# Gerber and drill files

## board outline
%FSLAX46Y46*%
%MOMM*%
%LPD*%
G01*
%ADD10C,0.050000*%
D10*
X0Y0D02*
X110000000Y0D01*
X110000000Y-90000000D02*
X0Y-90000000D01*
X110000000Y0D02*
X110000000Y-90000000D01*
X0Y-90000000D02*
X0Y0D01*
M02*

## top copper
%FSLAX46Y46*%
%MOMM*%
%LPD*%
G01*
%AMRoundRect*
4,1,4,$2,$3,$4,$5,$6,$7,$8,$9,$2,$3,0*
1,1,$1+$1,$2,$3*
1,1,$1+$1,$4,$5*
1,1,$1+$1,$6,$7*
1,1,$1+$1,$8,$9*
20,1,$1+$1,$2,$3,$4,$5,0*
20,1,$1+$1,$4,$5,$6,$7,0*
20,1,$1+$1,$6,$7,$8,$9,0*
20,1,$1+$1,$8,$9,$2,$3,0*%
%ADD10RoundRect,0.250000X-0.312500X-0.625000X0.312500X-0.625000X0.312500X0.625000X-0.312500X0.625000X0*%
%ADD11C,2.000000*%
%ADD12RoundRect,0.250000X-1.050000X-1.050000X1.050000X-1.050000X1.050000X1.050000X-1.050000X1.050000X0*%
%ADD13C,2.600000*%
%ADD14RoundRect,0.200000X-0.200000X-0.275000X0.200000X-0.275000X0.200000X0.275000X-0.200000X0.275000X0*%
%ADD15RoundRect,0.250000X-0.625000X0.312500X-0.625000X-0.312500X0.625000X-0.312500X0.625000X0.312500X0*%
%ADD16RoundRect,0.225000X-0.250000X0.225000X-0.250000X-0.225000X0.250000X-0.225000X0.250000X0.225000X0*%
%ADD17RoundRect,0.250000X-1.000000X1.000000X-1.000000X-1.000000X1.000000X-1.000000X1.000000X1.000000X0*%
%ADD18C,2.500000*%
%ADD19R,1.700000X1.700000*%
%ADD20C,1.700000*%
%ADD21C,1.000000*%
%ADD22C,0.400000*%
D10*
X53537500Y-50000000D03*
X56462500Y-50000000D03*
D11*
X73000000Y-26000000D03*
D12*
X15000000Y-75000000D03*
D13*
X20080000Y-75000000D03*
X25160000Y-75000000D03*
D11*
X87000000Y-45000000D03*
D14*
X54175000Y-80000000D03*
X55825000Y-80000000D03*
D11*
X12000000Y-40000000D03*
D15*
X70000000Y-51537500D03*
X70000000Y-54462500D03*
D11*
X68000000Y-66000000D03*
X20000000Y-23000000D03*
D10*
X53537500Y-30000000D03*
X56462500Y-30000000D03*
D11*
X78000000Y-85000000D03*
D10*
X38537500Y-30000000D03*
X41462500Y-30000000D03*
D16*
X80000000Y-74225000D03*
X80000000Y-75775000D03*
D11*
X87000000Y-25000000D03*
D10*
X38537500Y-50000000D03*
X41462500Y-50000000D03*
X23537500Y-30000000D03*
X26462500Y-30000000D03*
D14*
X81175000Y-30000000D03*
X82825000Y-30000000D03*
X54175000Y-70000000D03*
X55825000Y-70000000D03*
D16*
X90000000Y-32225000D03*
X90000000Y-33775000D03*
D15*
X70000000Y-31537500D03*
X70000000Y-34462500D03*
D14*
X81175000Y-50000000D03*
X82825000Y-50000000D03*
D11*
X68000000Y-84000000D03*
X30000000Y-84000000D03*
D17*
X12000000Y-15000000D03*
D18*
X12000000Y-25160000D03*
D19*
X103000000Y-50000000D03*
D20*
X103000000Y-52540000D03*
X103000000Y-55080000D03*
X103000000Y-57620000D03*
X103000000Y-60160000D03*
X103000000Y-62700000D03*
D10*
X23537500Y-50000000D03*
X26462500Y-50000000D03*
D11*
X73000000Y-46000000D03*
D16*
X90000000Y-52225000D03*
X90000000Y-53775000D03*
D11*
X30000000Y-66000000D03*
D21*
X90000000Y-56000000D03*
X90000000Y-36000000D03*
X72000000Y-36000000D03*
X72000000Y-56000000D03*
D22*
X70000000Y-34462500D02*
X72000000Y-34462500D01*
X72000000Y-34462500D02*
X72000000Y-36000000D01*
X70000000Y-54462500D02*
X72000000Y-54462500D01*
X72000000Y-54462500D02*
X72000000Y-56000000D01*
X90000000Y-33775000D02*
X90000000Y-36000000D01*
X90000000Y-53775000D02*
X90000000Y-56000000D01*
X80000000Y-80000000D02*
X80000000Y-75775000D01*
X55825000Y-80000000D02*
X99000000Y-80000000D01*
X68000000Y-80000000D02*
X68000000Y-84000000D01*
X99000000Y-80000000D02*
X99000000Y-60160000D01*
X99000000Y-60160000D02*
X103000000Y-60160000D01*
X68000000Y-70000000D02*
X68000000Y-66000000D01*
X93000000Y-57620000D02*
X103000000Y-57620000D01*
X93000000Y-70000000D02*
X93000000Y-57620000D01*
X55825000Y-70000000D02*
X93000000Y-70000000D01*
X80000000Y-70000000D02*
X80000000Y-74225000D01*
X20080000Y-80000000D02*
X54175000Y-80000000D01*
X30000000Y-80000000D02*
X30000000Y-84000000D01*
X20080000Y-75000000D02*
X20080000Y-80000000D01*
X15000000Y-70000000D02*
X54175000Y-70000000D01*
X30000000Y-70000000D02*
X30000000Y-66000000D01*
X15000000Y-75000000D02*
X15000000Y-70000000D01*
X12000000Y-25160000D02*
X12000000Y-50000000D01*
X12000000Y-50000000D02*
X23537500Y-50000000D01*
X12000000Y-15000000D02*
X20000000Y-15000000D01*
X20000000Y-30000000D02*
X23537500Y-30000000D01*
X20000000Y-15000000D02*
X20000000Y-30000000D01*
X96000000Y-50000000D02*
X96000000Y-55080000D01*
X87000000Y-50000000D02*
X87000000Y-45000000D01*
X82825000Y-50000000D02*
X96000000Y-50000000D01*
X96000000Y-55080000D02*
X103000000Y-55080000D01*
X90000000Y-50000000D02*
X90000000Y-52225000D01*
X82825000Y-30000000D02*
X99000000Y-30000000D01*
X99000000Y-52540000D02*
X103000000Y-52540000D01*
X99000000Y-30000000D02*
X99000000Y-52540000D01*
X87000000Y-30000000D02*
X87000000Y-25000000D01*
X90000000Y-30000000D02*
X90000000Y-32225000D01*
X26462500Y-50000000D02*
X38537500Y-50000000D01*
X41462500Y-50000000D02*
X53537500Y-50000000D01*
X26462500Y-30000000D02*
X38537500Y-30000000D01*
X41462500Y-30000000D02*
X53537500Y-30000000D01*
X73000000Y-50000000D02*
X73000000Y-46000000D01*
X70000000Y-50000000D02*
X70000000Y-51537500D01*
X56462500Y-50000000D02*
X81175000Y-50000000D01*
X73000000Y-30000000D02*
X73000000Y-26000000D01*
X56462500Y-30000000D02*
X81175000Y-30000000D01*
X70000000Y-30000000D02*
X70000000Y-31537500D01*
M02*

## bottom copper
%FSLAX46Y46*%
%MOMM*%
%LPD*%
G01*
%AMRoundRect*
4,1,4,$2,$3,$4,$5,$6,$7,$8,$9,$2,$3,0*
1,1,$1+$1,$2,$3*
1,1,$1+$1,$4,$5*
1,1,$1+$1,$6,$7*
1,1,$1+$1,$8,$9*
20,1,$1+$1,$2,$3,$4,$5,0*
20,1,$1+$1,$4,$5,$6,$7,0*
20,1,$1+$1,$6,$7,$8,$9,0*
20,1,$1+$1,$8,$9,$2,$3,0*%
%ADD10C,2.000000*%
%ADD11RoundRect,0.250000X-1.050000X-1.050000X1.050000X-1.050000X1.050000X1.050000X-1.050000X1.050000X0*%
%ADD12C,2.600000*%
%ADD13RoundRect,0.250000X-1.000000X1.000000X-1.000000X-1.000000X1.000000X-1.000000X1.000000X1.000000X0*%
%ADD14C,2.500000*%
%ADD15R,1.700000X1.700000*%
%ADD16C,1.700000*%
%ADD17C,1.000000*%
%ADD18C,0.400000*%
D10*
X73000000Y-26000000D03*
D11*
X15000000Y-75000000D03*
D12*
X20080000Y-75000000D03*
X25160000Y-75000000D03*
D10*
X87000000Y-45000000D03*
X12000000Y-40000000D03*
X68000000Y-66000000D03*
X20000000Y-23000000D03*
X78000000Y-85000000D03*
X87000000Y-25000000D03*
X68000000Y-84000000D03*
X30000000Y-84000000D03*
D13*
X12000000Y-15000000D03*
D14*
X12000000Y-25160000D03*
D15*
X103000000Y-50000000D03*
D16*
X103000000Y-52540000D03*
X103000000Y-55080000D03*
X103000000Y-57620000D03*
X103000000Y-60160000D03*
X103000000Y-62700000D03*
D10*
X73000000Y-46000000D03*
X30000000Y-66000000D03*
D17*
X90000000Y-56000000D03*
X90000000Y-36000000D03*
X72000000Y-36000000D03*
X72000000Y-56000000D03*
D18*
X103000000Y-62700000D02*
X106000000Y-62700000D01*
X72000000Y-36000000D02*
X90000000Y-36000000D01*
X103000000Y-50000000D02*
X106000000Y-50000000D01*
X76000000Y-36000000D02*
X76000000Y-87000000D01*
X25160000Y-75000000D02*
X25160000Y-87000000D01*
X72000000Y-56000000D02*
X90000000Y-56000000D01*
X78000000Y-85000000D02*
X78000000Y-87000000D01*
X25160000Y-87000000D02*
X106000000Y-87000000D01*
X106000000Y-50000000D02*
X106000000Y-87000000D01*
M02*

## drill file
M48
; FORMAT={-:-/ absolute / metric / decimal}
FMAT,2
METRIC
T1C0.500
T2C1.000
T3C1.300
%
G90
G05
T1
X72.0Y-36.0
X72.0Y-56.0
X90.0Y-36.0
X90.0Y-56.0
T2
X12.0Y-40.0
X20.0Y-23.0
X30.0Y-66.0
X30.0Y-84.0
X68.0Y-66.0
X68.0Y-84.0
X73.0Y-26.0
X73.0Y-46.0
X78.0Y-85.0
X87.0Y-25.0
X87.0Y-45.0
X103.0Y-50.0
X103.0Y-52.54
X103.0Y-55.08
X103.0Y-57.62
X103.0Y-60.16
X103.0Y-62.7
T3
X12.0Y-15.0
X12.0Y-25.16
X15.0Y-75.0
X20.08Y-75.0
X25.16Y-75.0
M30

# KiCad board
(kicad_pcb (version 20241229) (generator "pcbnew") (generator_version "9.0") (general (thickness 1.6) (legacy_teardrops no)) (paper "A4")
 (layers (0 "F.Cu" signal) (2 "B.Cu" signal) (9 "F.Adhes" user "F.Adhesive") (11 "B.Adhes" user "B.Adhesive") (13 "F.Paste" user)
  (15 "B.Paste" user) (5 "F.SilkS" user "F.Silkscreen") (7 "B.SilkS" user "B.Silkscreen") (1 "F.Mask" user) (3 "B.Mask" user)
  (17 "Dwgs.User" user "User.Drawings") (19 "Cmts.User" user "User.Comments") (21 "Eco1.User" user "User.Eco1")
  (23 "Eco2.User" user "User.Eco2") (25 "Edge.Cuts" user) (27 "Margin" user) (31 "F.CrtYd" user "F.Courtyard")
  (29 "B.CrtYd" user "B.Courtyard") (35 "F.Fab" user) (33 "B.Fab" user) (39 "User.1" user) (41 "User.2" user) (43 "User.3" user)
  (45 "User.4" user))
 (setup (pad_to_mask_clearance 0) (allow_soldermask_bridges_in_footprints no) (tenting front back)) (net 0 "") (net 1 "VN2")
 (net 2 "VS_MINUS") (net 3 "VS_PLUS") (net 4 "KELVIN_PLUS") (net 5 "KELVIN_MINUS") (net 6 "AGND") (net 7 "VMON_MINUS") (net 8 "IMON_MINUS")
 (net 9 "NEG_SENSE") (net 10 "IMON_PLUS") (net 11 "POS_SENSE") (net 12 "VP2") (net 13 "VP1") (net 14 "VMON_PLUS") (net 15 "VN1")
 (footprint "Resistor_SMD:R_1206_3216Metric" (layer "F.Cu") (at 55 50)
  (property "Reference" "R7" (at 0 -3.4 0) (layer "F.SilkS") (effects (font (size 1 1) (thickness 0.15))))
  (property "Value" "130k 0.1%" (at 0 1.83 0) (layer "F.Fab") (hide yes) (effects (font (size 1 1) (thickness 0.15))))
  (pad "1" smd roundrect (at -1.4625 0) (size 1.125 1.75) (layers "F.Cu" "F.Mask" "F.Paste") (roundrect_rratio 0.222222) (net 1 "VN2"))
  (pad "2" smd roundrect (at 1.4625 0) (size 1.125 1.75) (layers "F.Cu" "F.Mask" "F.Paste") (roundrect_rratio 0.222222) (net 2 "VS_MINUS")))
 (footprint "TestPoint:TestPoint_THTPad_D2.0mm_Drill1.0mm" (layer "F.Cu") (at 73 26)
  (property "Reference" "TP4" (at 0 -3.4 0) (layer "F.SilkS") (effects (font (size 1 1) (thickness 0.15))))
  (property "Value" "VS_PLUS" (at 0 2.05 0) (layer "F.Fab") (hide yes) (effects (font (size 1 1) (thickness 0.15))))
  (pad "1" thru_hole circle (at 0 0) (size 2 2) (drill 1) (layers "*.Cu" "*.Mask") (remove_unused_layers no) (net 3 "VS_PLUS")))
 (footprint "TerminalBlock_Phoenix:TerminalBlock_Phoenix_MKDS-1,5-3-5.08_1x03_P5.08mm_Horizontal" (layer "F.Cu") (at 15 75)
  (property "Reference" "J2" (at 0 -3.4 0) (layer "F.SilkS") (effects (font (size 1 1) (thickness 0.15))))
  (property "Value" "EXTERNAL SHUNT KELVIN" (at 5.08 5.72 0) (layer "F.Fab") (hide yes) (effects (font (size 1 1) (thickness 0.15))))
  (pad "1" thru_hole roundrect (at 0 0) (size 2.6 2.6) (drill 1.3) (layers "*.Cu" "*.Mask") (remove_unused_layers no)
   (roundrect_rratio 0.096154) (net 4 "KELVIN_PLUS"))
  (pad "2" thru_hole circle (at 5.08 0) (size 2.6 2.6) (drill 1.3) (layers "*.Cu" "*.Mask") (remove_unused_layers no) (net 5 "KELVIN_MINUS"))
  (pad "3" thru_hole circle (at 10.16 0) (size 2.6 2.6) (drill 1.3) (layers "*.Cu" "*.Mask") (remove_unused_layers no) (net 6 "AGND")))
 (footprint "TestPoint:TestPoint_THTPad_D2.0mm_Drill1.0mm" (layer "F.Cu") (at 87 45)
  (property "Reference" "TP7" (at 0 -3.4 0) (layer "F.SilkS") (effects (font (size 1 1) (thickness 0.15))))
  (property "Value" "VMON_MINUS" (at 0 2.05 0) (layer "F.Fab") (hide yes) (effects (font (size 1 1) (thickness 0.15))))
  (pad "1" thru_hole circle (at 0 0) (size 2 2) (drill 1) (layers "*.Cu" "*.Mask") (remove_unused_layers no) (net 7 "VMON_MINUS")))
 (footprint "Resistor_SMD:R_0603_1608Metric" (layer "F.Cu") (at 55 80)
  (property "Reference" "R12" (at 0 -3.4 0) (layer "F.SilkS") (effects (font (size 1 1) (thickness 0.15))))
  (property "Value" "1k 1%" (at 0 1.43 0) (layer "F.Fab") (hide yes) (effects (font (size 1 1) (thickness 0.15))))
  (pad "1" smd roundrect (at -0.825 0) (size 0.8 0.95) (layers "F.Cu" "F.Mask" "F.Paste") (roundrect_rratio 0.25) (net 5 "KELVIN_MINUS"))
  (pad "2" smd roundrect (at 0.825 0) (size 0.8 0.95) (layers "F.Cu" "F.Mask" "F.Paste") (roundrect_rratio 0.25) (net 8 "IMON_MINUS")))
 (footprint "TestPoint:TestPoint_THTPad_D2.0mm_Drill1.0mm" (layer "F.Cu") (at 12 40)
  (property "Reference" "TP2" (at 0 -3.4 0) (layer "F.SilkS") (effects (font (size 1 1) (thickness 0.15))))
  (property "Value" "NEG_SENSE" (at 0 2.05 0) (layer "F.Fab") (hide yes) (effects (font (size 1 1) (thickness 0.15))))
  (pad "1" thru_hole circle (at 0 0) (size 2 2) (drill 1) (layers "*.Cu" "*.Mask") (remove_unused_layers no) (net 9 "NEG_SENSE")))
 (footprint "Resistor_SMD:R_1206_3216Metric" (layer "F.Cu") (at 70 53 -90)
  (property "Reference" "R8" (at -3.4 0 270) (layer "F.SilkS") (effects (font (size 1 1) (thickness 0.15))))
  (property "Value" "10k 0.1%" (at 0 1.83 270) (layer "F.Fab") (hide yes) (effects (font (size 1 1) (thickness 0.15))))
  (pad "1" smd roundrect (at -1.4625 0 270) (size 1.125 1.75) (layers "F.Cu" "F.Mask" "F.Paste") (roundrect_rratio 0.222222)
   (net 2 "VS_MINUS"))
  (pad "2" smd roundrect (at 1.4625 0 270) (size 1.125 1.75) (layers "F.Cu" "F.Mask" "F.Paste") (roundrect_rratio 0.222222) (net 6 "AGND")))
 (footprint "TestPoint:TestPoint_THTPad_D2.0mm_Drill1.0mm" (layer "F.Cu") (at 68 66)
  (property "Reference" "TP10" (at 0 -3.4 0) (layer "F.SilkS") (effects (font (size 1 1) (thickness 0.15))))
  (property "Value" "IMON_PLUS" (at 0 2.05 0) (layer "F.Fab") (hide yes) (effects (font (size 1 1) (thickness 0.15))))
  (pad "1" thru_hole circle (at 0 0) (size 2 2) (drill 1) (layers "*.Cu" "*.Mask") (remove_unused_layers no) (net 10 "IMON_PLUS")))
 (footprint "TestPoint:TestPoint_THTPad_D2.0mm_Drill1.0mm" (layer "F.Cu") (at 20 23)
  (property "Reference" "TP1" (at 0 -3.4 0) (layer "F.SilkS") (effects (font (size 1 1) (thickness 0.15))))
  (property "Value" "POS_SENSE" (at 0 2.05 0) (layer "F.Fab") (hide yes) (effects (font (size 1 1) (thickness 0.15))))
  (pad "1" thru_hole circle (at 0 0) (size 2 2) (drill 1) (layers "*.Cu" "*.Mask") (remove_unused_layers no) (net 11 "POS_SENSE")))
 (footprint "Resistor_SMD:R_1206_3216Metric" (layer "F.Cu") (at 55 30)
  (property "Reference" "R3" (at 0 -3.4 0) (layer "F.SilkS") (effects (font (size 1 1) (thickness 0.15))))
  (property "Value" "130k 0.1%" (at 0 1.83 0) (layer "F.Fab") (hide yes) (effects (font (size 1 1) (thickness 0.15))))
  (pad "1" smd roundrect (at -1.4625 0) (size 1.125 1.75) (layers "F.Cu" "F.Mask" "F.Paste") (roundrect_rratio 0.222222) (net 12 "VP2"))
  (pad "2" smd roundrect (at 1.4625 0) (size 1.125 1.75) (layers "F.Cu" "F.Mask" "F.Paste") (roundrect_rratio 0.222222) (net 3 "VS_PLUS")))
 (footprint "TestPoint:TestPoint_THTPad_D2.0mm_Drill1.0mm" (layer "F.Cu") (at 78 85)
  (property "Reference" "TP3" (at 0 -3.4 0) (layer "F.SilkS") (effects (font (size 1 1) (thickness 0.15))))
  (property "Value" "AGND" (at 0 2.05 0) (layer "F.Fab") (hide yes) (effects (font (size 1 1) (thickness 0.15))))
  (pad "1" thru_hole circle (at 0 0) (size 2 2) (drill 1) (layers "*.Cu" "*.Mask") (remove_unused_layers no) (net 6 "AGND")))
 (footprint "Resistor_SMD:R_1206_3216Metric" (layer "F.Cu") (at 40 30)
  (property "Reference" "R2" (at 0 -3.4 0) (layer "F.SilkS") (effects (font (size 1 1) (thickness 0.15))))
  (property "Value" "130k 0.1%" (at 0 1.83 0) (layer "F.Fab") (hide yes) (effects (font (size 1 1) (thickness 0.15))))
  (pad "1" smd roundrect (at -1.4625 0) (size 1.125 1.75) (layers "F.Cu" "F.Mask" "F.Paste") (roundrect_rratio 0.222222) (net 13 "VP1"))
  (pad "2" smd roundrect (at 1.4625 0) (size 1.125 1.75) (layers "F.Cu" "F.Mask" "F.Paste") (roundrect_rratio 0.222222) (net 12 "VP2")))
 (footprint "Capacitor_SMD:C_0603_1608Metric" (layer "F.Cu") (at 80 75 -90)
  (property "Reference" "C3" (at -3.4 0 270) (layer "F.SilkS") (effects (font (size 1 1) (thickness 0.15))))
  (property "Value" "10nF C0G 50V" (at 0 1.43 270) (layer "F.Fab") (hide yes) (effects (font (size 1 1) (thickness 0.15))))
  (pad "1" smd roundrect (at -0.775 0 270) (size 0.9 0.95) (layers "F.Cu" "F.Mask" "F.Paste") (roundrect_rratio 0.25) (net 10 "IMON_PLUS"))
  (pad "2" smd roundrect (at 0.775 0 270) (size 0.9 0.95) (layers "F.Cu" "F.Mask" "F.Paste") (roundrect_rratio 0.25) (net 8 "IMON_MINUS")))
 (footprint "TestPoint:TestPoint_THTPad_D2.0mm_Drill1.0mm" (layer "F.Cu") (at 87 25)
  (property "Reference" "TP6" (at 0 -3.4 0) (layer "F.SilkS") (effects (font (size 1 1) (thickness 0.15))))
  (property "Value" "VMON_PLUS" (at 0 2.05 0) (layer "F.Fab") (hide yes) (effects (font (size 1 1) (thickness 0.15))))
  (pad "1" thru_hole circle (at 0 0) (size 2 2) (drill 1) (layers "*.Cu" "*.Mask") (remove_unused_layers no) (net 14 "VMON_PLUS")))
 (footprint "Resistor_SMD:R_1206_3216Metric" (layer "F.Cu") (at 40 50)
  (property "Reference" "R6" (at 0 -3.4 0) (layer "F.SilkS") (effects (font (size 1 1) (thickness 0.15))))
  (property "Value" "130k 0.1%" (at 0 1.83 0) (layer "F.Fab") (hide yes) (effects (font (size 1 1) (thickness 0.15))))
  (pad "1" smd roundrect (at -1.4625 0) (size 1.125 1.75) (layers "F.Cu" "F.Mask" "F.Paste") (roundrect_rratio 0.222222) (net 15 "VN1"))
  (pad "2" smd roundrect (at 1.4625 0) (size 1.125 1.75) (layers "F.Cu" "F.Mask" "F.Paste") (roundrect_rratio 0.222222) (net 1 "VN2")))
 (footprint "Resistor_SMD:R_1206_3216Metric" (layer "F.Cu") (at 25 30)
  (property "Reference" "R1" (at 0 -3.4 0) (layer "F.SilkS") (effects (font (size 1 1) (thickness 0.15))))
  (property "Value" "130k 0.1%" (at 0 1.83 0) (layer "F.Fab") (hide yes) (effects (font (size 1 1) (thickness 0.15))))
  (pad "1" smd roundrect (at -1.4625 0) (size 1.125 1.75) (layers "F.Cu" "F.Mask" "F.Paste") (roundrect_rratio 0.222222)
   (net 11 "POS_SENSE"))
  (pad "2" smd roundrect (at 1.4625 0) (size 1.125 1.75) (layers "F.Cu" "F.Mask" "F.Paste") (roundrect_rratio 0.222222) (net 13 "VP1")))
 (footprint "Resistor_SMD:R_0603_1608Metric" (layer "F.Cu") (at 82 30)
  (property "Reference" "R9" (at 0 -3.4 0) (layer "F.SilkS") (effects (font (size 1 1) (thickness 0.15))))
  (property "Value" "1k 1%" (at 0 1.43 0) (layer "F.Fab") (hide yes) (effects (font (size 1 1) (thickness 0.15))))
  (pad "1" smd roundrect (at -0.825 0) (size 0.8 0.95) (layers "F.Cu" "F.Mask" "F.Paste") (roundrect_rratio 0.25) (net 3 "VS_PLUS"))
  (pad "2" smd roundrect (at 0.825 0) (size 0.8 0.95) (layers "F.Cu" "F.Mask" "F.Paste") (roundrect_rratio 0.25) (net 14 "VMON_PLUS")))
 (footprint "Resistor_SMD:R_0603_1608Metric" (layer "F.Cu") (at 55 70)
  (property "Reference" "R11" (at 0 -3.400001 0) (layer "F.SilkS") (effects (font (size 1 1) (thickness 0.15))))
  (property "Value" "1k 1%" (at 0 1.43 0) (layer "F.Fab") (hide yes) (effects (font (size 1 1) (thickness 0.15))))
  (pad "1" smd roundrect (at -0.825 0) (size 0.8 0.95) (layers "F.Cu" "F.Mask" "F.Paste") (roundrect_rratio 0.25) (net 4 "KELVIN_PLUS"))
  (pad "2" smd roundrect (at 0.825 0) (size 0.8 0.95) (layers "F.Cu" "F.Mask" "F.Paste") (roundrect_rratio 0.25) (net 10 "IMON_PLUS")))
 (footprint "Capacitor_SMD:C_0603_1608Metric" (layer "F.Cu") (at 90 33 -90)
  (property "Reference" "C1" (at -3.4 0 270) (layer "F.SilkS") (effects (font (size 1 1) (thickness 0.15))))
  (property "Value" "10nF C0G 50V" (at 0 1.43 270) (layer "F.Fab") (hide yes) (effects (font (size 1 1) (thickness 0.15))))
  (pad "1" smd roundrect (at -0.775 0 270) (size 0.9 0.95) (layers "F.Cu" "F.Mask" "F.Paste") (roundrect_rratio 0.25) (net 14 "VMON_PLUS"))
  (pad "2" smd roundrect (at 0.775 0 270) (size 0.9 0.95) (layers "F.Cu" "F.Mask" "F.Paste") (roundrect_rratio 0.25) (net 6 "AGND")))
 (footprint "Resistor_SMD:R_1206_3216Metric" (layer "F.Cu") (at 70 33 -90)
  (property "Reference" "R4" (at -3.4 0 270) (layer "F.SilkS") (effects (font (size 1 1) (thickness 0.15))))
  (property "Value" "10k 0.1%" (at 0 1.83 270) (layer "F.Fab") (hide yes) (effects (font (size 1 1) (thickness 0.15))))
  (pad "1" smd roundrect (at -1.4625 0 270) (size 1.125 1.75) (layers "F.Cu" "F.Mask" "F.Paste") (roundrect_rratio 0.222222)
   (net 3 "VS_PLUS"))
  (pad "2" smd roundrect (at 1.4625 0 270) (size 1.125 1.75) (layers "F.Cu" "F.Mask" "F.Paste") (roundrect_rratio 0.222222) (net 6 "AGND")))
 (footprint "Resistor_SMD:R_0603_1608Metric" (layer "F.Cu") (at 82 50)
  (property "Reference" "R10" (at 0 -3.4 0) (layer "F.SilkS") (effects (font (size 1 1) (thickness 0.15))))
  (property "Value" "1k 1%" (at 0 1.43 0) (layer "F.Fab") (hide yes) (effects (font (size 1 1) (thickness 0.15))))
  (pad "1" smd roundrect (at -0.825 0) (size 0.8 0.95) (layers "F.Cu" "F.Mask" "F.Paste") (roundrect_rratio 0.25) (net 2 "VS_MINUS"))
  (pad "2" smd roundrect (at 0.825 0) (size 0.8 0.95) (layers "F.Cu" "F.Mask" "F.Paste") (roundrect_rratio 0.25) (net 7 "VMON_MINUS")))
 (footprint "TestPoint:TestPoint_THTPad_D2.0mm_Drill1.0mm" (layer "F.Cu") (at 68 84)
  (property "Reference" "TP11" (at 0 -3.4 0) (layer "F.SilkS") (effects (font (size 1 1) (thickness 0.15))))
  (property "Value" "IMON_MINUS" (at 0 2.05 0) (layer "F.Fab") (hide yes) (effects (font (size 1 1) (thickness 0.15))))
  (pad "1" thru_hole circle (at 0 0) (size 2 2) (drill 1) (layers "*.Cu" "*.Mask") (remove_unused_layers no) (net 8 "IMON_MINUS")))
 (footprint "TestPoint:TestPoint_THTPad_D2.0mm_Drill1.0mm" (layer "F.Cu") (at 30 84)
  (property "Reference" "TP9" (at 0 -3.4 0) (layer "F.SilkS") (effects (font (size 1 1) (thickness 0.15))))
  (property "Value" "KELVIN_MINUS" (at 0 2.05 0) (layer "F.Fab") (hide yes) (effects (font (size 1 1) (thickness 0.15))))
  (pad "1" thru_hole circle (at 0 0) (size 2 2) (drill 1) (layers "*.Cu" "*.Mask") (remove_unused_layers no) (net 5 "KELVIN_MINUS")))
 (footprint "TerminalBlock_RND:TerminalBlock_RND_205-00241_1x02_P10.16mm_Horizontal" (layer "F.Cu") (at 12 15 -90)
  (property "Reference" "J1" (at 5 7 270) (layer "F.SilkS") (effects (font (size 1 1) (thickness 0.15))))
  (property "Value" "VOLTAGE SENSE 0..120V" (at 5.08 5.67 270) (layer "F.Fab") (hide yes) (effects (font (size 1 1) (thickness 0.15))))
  (pad "1" thru_hole roundrect (at 0 0 270) (size 2.5 2.5) (drill 1.3) (layers "*.Cu" "*.Mask") (remove_unused_layers no)
   (roundrect_rratio 0.1) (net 11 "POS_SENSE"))
  (pad "2" thru_hole circle (at 10.16 0 270) (size 2.5 2.5) (drill 1.3) (layers "*.Cu" "*.Mask") (remove_unused_layers no)
   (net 9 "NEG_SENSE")))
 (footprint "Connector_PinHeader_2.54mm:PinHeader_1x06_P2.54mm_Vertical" (layer "F.Cu") (at 103 50)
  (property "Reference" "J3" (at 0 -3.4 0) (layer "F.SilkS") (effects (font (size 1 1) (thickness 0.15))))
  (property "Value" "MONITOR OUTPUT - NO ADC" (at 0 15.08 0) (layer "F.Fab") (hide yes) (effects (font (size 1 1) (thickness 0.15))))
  (pad "1" thru_hole rect (at 0 0) (size 1.7 1.7) (drill 1) (layers "*.Cu" "*.Mask") (remove_unused_layers no) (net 6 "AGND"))
  (pad "2" thru_hole circle (at 0 2.54) (size 1.7 1.7) (drill 1) (layers "*.Cu" "*.Mask") (remove_unused_layers no) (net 14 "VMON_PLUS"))
  (pad "3" thru_hole circle (at 0 5.08) (size 1.7 1.7) (drill 1) (layers "*.Cu" "*.Mask") (remove_unused_layers no) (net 7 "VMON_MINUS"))
  (pad "4" thru_hole circle (at 0 7.62) (size 1.7 1.7) (drill 1) (layers "*.Cu" "*.Mask") (remove_unused_layers no) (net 10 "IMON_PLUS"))
  (pad "5" thru_hole circle (at 0 10.16) (size 1.7 1.7) (drill 1) (layers "*.Cu" "*.Mask") (remove_unused_layers no) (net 8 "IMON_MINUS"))
  (pad "6" thru_hole circle (at 0 12.7) (size 1.7 1.7) (drill 1) (layers "*.Cu" "*.Mask") (remove_unused_layers no) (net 6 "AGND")))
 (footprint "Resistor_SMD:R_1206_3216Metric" (layer "F.Cu") (at 25 50)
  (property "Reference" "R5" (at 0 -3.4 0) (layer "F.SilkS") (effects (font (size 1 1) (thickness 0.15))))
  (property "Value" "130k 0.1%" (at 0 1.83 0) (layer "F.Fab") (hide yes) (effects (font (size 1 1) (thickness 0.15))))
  (pad "1" smd roundrect (at -1.4625 0) (size 1.125 1.75) (layers "F.Cu" "F.Mask" "F.Paste") (roundrect_rratio 0.222222) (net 9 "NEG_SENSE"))
  (pad "2" smd roundrect (at 1.4625 0) (size 1.125 1.75) (layers "F.Cu" "F.Mask" "F.Paste") (roundrect_rratio 0.222222) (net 15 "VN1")))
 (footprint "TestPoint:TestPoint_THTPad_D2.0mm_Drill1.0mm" (layer "F.Cu") (at 73 46)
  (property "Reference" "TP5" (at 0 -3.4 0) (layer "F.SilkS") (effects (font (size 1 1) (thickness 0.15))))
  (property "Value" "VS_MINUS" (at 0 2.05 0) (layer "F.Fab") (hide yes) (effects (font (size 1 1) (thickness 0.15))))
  (pad "1" thru_hole circle (at 0 0) (size 2 2) (drill 1) (layers "*.Cu" "*.Mask") (remove_unused_layers no) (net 2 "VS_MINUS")))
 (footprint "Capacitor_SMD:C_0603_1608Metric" (layer "F.Cu") (at 90 53 -90)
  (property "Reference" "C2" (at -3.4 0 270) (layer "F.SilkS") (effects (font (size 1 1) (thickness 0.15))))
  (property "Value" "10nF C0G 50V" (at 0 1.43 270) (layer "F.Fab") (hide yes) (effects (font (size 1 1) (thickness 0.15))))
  (pad "1" smd roundrect (at -0.775 0 270) (size 0.9 0.95) (layers "F.Cu" "F.Mask" "F.Paste") (roundrect_rratio 0.25) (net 7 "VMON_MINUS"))
  (pad "2" smd roundrect (at 0.775 0 270) (size 0.9 0.95) (layers "F.Cu" "F.Mask" "F.Paste") (roundrect_rratio 0.25) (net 6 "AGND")))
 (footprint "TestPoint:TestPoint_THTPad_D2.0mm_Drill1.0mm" (layer "F.Cu") (at 30 66)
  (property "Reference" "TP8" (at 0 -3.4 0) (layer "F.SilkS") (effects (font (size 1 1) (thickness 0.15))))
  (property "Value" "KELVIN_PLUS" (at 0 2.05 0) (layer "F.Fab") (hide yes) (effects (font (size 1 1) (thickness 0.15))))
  (pad "1" thru_hole circle (at 0 0) (size 2 2) (drill 1) (layers "*.Cu" "*.Mask") (remove_unused_layers no) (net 4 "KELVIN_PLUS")))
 (gr_line (start 0 0) (end 110 0) (stroke (width 0.05) (type default)) (layer "Edge.Cuts"))
 (gr_line (start 110 90) (end 0 90) (stroke (width 0.05) (type default)) (layer "Edge.Cuts"))
 (gr_line (start 110 0) (end 110 90) (stroke (width 0.05) (type default)) (layer "Edge.Cuts"))
 (gr_line (start 0 90) (end 0 0) (stroke (width 0.05) (type default)) (layer "Edge.Cuts"))
 (segment (start 70 34.4625) (end 72 34.4625) (width 0.4) (layer "F.Cu") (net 6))
 (segment (start 72 34.4625) (end 72 36) (width 0.4) (layer "F.Cu") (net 6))
 (segment (start 70 54.4625) (end 72 54.4625) (width 0.4) (layer "F.Cu") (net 6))
 (segment (start 72 54.4625) (end 72 56) (width 0.4) (layer "F.Cu") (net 6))
 (segment (start 90 33.775) (end 90 36) (width 0.4) (layer "F.Cu") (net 6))
 (segment (start 90 53.775) (end 90 56) (width 0.4) (layer "F.Cu") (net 6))
 (via (at 90 56) (size 1) (drill 0.5) (layers "F.Cu" "B.Cu") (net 6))
 (via (at 90 36) (size 1) (drill 0.5) (layers "F.Cu" "B.Cu") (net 6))
 (via (at 72 36) (size 1) (drill 0.5) (layers "F.Cu" "B.Cu") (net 6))
 (via (at 72 56) (size 1) (drill 0.5) (layers "F.Cu" "B.Cu") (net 6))
 (segment (start 103 62.7) (end 106 62.7) (width 0.4) (layer "B.Cu") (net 6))
 (segment (start 72 36) (end 90 36) (width 0.4) (layer "B.Cu") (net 6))
 (segment (start 103 50) (end 106 50) (width 0.4) (layer "B.Cu") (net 6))
 (segment (start 76 36) (end 76 87) (width 0.4) (layer "B.Cu") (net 6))
 (segment (start 25.16 75) (end 25.16 87) (width 0.4) (layer "B.Cu") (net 6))
 (segment (start 72 56) (end 90 56) (width 0.4) (layer "B.Cu") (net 6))
 (segment (start 78 85) (end 78 87) (width 0.4) (layer "B.Cu") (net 6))
 (segment (start 25.16 87) (end 106 87) (width 0.4) (layer "B.Cu") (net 6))
 (segment (start 106 50) (end 106 87) (width 0.4) (layer "B.Cu") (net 6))
 (segment (start 80 80) (end 80 75.775) (width 0.4) (layer "F.Cu") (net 8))
 (segment (start 55.825 80) (end 99 80) (width 0.4) (layer "F.Cu") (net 8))
 (segment (start 68 80) (end 68 84) (width 0.4) (layer "F.Cu") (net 8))
 (segment (start 99 80) (end 99 60.16) (width 0.4) (layer "F.Cu") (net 8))
 (segment (start 99 60.16) (end 103 60.16) (width 0.4) (layer "F.Cu") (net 8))
 (segment (start 68 70) (end 68 66) (width 0.4) (layer "F.Cu") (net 10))
 (segment (start 93 57.62) (end 103 57.62) (width 0.4) (layer "F.Cu") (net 10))
 (segment (start 93 70) (end 93 57.62) (width 0.4) (layer "F.Cu") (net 10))
 (segment (start 55.825 70) (end 93 70) (width 0.4) (layer "F.Cu") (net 10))
 (segment (start 80 70) (end 80 74.225) (width 0.4) (layer "F.Cu") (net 10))
 (segment (start 20.08 80) (end 54.175 80) (width 0.4) (layer "F.Cu") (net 5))
 (segment (start 30 80) (end 30 84) (width 0.4) (layer "F.Cu") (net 5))
 (segment (start 20.08 75) (end 20.08 80) (width 0.4) (layer "F.Cu") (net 5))
 (segment (start 15 70) (end 54.175 70) (width 0.4) (layer "F.Cu") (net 4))
 (segment (start 30 70) (end 30 66) (width 0.4) (layer "F.Cu") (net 4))
 (segment (start 15 75) (end 15 70) (width 0.4) (layer "F.Cu") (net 4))
 (segment (start 12 25.16) (end 12 50) (width 0.4) (layer "F.Cu") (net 9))
 (segment (start 12 50) (end 23.5375 50) (width 0.4) (layer "F.Cu") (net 9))
 (segment (start 12 15) (end 20 15) (width 0.4) (layer "F.Cu") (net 11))
 (segment (start 20 30) (end 23.5375 30) (width 0.4) (layer "F.Cu") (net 11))
 (segment (start 20 15) (end 20 30) (width 0.4) (layer "F.Cu") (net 11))
 (segment (start 96 50) (end 96 55.08) (width 0.4) (layer "F.Cu") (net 7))
 (segment (start 87 50) (end 87 45) (width 0.4) (layer "F.Cu") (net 7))
 (segment (start 82.825 50) (end 96 50) (width 0.4) (layer "F.Cu") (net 7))
 (segment (start 96 55.08) (end 103 55.08) (width 0.4) (layer "F.Cu") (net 7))
 (segment (start 90 50) (end 90 52.225) (width 0.4) (layer "F.Cu") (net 7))
 (segment (start 82.825 30) (end 99 30) (width 0.4) (layer "F.Cu") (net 14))
 (segment (start 99 52.54) (end 103 52.54) (width 0.4) (layer "F.Cu") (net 14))
 (segment (start 99 30) (end 99 52.54) (width 0.4) (layer "F.Cu") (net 14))
 (segment (start 87 30) (end 87 25) (width 0.4) (layer "F.Cu") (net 14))
 (segment (start 90 30) (end 90 32.225) (width 0.4) (layer "F.Cu") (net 14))
 (segment (start 26.4625 50) (end 38.5375 50) (width 0.4) (layer "F.Cu") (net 15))
 (segment (start 41.4625 50) (end 53.5375 50) (width 0.4) (layer "F.Cu") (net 1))
 (segment (start 26.4625 30) (end 38.5375 30) (width 0.4) (layer "F.Cu") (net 13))
 (segment (start 41.4625 30) (end 53.5375 30) (width 0.4) (layer "F.Cu") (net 12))
 (segment (start 73 50) (end 73 46) (width 0.4) (layer "F.Cu") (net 2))
 (segment (start 70 50) (end 70 51.5375) (width 0.4) (layer "F.Cu") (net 2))
 (segment (start 56.4625 50) (end 81.175 50) (width 0.4) (layer "F.Cu") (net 2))
 (segment (start 73 30) (end 73 26) (width 0.4) (layer "F.Cu") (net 3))
 (segment (start 56.4625 30) (end 81.175 30) (width 0.4) (layer "F.Cu") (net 3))
 (segment (start 70 30) (end 70 31.5375) (width 0.4) (layer "F.Cu") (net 3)))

